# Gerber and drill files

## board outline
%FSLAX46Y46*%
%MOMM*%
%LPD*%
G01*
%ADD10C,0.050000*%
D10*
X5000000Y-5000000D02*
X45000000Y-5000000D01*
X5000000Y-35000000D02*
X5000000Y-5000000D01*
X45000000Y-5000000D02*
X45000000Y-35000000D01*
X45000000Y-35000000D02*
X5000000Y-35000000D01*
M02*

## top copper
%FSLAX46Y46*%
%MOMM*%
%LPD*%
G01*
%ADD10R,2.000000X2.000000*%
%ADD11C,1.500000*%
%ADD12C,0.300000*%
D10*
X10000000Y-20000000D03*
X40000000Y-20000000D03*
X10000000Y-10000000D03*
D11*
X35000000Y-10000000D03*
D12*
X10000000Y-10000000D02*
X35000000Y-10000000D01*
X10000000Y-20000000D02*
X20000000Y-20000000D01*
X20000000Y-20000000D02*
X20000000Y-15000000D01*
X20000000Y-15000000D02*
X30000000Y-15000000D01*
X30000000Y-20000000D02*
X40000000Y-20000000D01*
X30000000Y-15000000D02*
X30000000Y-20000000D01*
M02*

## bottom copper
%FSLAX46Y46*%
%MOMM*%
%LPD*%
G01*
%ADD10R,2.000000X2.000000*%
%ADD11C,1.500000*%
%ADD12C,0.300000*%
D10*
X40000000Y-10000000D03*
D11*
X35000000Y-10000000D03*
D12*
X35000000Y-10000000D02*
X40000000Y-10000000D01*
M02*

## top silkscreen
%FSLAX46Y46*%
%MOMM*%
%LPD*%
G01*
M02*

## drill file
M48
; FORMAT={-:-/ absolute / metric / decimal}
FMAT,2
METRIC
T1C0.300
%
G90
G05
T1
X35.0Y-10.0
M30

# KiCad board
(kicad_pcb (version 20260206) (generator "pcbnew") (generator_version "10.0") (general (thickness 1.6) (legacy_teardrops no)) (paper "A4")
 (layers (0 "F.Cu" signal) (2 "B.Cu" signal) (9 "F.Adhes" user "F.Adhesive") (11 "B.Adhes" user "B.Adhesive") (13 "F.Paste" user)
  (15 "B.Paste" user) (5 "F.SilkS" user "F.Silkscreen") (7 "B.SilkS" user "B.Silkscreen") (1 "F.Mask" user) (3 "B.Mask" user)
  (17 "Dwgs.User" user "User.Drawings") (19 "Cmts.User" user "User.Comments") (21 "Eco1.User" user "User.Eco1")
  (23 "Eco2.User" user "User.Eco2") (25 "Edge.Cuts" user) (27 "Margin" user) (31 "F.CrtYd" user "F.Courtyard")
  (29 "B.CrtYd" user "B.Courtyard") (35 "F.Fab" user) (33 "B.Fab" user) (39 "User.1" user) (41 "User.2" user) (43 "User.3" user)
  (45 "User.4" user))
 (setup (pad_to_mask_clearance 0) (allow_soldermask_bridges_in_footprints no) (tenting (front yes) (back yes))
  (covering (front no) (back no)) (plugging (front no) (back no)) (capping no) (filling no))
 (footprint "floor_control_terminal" (layer "F.Cu") (at 10 20)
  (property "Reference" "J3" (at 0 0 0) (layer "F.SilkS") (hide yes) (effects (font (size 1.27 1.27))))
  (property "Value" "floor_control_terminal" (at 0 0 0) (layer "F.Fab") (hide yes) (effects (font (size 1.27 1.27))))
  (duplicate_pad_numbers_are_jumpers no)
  (pad "1" smd rect (at 0 0) (size 2 2) (layers "F.Cu" "F.Mask" "F.Paste") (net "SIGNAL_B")))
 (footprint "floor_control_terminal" (layer "F.Cu") (at 40 20)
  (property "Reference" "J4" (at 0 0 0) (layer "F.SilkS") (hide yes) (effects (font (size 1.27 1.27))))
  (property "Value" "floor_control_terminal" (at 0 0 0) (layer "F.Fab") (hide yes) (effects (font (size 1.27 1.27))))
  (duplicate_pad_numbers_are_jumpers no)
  (pad "1" smd rect (at 0 0) (size 2 2) (layers "F.Cu" "F.Mask" "F.Paste") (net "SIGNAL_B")))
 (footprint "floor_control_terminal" (layer "F.Cu") (at 10 10)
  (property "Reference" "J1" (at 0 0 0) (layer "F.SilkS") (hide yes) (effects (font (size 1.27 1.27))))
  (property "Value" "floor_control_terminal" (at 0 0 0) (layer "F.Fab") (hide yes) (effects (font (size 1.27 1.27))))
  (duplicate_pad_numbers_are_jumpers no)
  (pad "1" smd rect (at 0 0) (size 2 2) (layers "F.Cu" "F.Mask" "F.Paste") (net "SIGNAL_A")))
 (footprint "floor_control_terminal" (layer "B.Cu") (at 40 10)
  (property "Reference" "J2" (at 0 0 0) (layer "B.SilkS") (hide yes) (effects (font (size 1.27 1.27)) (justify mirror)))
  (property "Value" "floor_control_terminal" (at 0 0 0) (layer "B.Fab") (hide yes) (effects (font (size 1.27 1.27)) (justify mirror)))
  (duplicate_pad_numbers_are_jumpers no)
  (pad "1" smd rect (at 0 0) (size 2 2) (layers "B.Cu" "B.Mask" "B.Paste") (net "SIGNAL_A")))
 (gr_line (start 5 5) (end 45 5) (stroke (width 0.05) (type default)) (layer "Edge.Cuts"))
 (gr_line (start 5 35) (end 5 5) (stroke (width 0.05) (type default)) (layer "Edge.Cuts"))
 (gr_line (start 45 5) (end 45 35) (stroke (width 0.05) (type default)) (layer "Edge.Cuts"))
 (gr_line (start 45 35) (end 5 35) (stroke (width 0.05) (type default)) (layer "Edge.Cuts"))
 (segment (start 10 10) (end 35 10) (width 0.3) (layer "F.Cu") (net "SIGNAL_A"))
 (via (at 35 10) (size 1.5) (drill 0.3) (layers "F.Cu" "B.Cu") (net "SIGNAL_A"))
 (segment (start 35 10) (end 40 10) (width 0.3) (layer "B.Cu") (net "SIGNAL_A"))
 (segment (start 10 20) (end 20 20) (width 0.3) (layer "F.Cu") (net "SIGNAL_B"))
 (segment (start 20 20) (end 20 15) (width 0.3) (layer "F.Cu") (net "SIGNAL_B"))
 (segment (start 20 15) (end 30 15) (width 0.3) (layer "F.Cu") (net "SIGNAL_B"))
 (segment (start 30 20) (end 40 20) (width 0.3) (layer "F.Cu") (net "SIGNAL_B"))
 (segment (start 30 15) (end 30 20) (width 0.3) (layer "F.Cu") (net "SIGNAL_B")))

